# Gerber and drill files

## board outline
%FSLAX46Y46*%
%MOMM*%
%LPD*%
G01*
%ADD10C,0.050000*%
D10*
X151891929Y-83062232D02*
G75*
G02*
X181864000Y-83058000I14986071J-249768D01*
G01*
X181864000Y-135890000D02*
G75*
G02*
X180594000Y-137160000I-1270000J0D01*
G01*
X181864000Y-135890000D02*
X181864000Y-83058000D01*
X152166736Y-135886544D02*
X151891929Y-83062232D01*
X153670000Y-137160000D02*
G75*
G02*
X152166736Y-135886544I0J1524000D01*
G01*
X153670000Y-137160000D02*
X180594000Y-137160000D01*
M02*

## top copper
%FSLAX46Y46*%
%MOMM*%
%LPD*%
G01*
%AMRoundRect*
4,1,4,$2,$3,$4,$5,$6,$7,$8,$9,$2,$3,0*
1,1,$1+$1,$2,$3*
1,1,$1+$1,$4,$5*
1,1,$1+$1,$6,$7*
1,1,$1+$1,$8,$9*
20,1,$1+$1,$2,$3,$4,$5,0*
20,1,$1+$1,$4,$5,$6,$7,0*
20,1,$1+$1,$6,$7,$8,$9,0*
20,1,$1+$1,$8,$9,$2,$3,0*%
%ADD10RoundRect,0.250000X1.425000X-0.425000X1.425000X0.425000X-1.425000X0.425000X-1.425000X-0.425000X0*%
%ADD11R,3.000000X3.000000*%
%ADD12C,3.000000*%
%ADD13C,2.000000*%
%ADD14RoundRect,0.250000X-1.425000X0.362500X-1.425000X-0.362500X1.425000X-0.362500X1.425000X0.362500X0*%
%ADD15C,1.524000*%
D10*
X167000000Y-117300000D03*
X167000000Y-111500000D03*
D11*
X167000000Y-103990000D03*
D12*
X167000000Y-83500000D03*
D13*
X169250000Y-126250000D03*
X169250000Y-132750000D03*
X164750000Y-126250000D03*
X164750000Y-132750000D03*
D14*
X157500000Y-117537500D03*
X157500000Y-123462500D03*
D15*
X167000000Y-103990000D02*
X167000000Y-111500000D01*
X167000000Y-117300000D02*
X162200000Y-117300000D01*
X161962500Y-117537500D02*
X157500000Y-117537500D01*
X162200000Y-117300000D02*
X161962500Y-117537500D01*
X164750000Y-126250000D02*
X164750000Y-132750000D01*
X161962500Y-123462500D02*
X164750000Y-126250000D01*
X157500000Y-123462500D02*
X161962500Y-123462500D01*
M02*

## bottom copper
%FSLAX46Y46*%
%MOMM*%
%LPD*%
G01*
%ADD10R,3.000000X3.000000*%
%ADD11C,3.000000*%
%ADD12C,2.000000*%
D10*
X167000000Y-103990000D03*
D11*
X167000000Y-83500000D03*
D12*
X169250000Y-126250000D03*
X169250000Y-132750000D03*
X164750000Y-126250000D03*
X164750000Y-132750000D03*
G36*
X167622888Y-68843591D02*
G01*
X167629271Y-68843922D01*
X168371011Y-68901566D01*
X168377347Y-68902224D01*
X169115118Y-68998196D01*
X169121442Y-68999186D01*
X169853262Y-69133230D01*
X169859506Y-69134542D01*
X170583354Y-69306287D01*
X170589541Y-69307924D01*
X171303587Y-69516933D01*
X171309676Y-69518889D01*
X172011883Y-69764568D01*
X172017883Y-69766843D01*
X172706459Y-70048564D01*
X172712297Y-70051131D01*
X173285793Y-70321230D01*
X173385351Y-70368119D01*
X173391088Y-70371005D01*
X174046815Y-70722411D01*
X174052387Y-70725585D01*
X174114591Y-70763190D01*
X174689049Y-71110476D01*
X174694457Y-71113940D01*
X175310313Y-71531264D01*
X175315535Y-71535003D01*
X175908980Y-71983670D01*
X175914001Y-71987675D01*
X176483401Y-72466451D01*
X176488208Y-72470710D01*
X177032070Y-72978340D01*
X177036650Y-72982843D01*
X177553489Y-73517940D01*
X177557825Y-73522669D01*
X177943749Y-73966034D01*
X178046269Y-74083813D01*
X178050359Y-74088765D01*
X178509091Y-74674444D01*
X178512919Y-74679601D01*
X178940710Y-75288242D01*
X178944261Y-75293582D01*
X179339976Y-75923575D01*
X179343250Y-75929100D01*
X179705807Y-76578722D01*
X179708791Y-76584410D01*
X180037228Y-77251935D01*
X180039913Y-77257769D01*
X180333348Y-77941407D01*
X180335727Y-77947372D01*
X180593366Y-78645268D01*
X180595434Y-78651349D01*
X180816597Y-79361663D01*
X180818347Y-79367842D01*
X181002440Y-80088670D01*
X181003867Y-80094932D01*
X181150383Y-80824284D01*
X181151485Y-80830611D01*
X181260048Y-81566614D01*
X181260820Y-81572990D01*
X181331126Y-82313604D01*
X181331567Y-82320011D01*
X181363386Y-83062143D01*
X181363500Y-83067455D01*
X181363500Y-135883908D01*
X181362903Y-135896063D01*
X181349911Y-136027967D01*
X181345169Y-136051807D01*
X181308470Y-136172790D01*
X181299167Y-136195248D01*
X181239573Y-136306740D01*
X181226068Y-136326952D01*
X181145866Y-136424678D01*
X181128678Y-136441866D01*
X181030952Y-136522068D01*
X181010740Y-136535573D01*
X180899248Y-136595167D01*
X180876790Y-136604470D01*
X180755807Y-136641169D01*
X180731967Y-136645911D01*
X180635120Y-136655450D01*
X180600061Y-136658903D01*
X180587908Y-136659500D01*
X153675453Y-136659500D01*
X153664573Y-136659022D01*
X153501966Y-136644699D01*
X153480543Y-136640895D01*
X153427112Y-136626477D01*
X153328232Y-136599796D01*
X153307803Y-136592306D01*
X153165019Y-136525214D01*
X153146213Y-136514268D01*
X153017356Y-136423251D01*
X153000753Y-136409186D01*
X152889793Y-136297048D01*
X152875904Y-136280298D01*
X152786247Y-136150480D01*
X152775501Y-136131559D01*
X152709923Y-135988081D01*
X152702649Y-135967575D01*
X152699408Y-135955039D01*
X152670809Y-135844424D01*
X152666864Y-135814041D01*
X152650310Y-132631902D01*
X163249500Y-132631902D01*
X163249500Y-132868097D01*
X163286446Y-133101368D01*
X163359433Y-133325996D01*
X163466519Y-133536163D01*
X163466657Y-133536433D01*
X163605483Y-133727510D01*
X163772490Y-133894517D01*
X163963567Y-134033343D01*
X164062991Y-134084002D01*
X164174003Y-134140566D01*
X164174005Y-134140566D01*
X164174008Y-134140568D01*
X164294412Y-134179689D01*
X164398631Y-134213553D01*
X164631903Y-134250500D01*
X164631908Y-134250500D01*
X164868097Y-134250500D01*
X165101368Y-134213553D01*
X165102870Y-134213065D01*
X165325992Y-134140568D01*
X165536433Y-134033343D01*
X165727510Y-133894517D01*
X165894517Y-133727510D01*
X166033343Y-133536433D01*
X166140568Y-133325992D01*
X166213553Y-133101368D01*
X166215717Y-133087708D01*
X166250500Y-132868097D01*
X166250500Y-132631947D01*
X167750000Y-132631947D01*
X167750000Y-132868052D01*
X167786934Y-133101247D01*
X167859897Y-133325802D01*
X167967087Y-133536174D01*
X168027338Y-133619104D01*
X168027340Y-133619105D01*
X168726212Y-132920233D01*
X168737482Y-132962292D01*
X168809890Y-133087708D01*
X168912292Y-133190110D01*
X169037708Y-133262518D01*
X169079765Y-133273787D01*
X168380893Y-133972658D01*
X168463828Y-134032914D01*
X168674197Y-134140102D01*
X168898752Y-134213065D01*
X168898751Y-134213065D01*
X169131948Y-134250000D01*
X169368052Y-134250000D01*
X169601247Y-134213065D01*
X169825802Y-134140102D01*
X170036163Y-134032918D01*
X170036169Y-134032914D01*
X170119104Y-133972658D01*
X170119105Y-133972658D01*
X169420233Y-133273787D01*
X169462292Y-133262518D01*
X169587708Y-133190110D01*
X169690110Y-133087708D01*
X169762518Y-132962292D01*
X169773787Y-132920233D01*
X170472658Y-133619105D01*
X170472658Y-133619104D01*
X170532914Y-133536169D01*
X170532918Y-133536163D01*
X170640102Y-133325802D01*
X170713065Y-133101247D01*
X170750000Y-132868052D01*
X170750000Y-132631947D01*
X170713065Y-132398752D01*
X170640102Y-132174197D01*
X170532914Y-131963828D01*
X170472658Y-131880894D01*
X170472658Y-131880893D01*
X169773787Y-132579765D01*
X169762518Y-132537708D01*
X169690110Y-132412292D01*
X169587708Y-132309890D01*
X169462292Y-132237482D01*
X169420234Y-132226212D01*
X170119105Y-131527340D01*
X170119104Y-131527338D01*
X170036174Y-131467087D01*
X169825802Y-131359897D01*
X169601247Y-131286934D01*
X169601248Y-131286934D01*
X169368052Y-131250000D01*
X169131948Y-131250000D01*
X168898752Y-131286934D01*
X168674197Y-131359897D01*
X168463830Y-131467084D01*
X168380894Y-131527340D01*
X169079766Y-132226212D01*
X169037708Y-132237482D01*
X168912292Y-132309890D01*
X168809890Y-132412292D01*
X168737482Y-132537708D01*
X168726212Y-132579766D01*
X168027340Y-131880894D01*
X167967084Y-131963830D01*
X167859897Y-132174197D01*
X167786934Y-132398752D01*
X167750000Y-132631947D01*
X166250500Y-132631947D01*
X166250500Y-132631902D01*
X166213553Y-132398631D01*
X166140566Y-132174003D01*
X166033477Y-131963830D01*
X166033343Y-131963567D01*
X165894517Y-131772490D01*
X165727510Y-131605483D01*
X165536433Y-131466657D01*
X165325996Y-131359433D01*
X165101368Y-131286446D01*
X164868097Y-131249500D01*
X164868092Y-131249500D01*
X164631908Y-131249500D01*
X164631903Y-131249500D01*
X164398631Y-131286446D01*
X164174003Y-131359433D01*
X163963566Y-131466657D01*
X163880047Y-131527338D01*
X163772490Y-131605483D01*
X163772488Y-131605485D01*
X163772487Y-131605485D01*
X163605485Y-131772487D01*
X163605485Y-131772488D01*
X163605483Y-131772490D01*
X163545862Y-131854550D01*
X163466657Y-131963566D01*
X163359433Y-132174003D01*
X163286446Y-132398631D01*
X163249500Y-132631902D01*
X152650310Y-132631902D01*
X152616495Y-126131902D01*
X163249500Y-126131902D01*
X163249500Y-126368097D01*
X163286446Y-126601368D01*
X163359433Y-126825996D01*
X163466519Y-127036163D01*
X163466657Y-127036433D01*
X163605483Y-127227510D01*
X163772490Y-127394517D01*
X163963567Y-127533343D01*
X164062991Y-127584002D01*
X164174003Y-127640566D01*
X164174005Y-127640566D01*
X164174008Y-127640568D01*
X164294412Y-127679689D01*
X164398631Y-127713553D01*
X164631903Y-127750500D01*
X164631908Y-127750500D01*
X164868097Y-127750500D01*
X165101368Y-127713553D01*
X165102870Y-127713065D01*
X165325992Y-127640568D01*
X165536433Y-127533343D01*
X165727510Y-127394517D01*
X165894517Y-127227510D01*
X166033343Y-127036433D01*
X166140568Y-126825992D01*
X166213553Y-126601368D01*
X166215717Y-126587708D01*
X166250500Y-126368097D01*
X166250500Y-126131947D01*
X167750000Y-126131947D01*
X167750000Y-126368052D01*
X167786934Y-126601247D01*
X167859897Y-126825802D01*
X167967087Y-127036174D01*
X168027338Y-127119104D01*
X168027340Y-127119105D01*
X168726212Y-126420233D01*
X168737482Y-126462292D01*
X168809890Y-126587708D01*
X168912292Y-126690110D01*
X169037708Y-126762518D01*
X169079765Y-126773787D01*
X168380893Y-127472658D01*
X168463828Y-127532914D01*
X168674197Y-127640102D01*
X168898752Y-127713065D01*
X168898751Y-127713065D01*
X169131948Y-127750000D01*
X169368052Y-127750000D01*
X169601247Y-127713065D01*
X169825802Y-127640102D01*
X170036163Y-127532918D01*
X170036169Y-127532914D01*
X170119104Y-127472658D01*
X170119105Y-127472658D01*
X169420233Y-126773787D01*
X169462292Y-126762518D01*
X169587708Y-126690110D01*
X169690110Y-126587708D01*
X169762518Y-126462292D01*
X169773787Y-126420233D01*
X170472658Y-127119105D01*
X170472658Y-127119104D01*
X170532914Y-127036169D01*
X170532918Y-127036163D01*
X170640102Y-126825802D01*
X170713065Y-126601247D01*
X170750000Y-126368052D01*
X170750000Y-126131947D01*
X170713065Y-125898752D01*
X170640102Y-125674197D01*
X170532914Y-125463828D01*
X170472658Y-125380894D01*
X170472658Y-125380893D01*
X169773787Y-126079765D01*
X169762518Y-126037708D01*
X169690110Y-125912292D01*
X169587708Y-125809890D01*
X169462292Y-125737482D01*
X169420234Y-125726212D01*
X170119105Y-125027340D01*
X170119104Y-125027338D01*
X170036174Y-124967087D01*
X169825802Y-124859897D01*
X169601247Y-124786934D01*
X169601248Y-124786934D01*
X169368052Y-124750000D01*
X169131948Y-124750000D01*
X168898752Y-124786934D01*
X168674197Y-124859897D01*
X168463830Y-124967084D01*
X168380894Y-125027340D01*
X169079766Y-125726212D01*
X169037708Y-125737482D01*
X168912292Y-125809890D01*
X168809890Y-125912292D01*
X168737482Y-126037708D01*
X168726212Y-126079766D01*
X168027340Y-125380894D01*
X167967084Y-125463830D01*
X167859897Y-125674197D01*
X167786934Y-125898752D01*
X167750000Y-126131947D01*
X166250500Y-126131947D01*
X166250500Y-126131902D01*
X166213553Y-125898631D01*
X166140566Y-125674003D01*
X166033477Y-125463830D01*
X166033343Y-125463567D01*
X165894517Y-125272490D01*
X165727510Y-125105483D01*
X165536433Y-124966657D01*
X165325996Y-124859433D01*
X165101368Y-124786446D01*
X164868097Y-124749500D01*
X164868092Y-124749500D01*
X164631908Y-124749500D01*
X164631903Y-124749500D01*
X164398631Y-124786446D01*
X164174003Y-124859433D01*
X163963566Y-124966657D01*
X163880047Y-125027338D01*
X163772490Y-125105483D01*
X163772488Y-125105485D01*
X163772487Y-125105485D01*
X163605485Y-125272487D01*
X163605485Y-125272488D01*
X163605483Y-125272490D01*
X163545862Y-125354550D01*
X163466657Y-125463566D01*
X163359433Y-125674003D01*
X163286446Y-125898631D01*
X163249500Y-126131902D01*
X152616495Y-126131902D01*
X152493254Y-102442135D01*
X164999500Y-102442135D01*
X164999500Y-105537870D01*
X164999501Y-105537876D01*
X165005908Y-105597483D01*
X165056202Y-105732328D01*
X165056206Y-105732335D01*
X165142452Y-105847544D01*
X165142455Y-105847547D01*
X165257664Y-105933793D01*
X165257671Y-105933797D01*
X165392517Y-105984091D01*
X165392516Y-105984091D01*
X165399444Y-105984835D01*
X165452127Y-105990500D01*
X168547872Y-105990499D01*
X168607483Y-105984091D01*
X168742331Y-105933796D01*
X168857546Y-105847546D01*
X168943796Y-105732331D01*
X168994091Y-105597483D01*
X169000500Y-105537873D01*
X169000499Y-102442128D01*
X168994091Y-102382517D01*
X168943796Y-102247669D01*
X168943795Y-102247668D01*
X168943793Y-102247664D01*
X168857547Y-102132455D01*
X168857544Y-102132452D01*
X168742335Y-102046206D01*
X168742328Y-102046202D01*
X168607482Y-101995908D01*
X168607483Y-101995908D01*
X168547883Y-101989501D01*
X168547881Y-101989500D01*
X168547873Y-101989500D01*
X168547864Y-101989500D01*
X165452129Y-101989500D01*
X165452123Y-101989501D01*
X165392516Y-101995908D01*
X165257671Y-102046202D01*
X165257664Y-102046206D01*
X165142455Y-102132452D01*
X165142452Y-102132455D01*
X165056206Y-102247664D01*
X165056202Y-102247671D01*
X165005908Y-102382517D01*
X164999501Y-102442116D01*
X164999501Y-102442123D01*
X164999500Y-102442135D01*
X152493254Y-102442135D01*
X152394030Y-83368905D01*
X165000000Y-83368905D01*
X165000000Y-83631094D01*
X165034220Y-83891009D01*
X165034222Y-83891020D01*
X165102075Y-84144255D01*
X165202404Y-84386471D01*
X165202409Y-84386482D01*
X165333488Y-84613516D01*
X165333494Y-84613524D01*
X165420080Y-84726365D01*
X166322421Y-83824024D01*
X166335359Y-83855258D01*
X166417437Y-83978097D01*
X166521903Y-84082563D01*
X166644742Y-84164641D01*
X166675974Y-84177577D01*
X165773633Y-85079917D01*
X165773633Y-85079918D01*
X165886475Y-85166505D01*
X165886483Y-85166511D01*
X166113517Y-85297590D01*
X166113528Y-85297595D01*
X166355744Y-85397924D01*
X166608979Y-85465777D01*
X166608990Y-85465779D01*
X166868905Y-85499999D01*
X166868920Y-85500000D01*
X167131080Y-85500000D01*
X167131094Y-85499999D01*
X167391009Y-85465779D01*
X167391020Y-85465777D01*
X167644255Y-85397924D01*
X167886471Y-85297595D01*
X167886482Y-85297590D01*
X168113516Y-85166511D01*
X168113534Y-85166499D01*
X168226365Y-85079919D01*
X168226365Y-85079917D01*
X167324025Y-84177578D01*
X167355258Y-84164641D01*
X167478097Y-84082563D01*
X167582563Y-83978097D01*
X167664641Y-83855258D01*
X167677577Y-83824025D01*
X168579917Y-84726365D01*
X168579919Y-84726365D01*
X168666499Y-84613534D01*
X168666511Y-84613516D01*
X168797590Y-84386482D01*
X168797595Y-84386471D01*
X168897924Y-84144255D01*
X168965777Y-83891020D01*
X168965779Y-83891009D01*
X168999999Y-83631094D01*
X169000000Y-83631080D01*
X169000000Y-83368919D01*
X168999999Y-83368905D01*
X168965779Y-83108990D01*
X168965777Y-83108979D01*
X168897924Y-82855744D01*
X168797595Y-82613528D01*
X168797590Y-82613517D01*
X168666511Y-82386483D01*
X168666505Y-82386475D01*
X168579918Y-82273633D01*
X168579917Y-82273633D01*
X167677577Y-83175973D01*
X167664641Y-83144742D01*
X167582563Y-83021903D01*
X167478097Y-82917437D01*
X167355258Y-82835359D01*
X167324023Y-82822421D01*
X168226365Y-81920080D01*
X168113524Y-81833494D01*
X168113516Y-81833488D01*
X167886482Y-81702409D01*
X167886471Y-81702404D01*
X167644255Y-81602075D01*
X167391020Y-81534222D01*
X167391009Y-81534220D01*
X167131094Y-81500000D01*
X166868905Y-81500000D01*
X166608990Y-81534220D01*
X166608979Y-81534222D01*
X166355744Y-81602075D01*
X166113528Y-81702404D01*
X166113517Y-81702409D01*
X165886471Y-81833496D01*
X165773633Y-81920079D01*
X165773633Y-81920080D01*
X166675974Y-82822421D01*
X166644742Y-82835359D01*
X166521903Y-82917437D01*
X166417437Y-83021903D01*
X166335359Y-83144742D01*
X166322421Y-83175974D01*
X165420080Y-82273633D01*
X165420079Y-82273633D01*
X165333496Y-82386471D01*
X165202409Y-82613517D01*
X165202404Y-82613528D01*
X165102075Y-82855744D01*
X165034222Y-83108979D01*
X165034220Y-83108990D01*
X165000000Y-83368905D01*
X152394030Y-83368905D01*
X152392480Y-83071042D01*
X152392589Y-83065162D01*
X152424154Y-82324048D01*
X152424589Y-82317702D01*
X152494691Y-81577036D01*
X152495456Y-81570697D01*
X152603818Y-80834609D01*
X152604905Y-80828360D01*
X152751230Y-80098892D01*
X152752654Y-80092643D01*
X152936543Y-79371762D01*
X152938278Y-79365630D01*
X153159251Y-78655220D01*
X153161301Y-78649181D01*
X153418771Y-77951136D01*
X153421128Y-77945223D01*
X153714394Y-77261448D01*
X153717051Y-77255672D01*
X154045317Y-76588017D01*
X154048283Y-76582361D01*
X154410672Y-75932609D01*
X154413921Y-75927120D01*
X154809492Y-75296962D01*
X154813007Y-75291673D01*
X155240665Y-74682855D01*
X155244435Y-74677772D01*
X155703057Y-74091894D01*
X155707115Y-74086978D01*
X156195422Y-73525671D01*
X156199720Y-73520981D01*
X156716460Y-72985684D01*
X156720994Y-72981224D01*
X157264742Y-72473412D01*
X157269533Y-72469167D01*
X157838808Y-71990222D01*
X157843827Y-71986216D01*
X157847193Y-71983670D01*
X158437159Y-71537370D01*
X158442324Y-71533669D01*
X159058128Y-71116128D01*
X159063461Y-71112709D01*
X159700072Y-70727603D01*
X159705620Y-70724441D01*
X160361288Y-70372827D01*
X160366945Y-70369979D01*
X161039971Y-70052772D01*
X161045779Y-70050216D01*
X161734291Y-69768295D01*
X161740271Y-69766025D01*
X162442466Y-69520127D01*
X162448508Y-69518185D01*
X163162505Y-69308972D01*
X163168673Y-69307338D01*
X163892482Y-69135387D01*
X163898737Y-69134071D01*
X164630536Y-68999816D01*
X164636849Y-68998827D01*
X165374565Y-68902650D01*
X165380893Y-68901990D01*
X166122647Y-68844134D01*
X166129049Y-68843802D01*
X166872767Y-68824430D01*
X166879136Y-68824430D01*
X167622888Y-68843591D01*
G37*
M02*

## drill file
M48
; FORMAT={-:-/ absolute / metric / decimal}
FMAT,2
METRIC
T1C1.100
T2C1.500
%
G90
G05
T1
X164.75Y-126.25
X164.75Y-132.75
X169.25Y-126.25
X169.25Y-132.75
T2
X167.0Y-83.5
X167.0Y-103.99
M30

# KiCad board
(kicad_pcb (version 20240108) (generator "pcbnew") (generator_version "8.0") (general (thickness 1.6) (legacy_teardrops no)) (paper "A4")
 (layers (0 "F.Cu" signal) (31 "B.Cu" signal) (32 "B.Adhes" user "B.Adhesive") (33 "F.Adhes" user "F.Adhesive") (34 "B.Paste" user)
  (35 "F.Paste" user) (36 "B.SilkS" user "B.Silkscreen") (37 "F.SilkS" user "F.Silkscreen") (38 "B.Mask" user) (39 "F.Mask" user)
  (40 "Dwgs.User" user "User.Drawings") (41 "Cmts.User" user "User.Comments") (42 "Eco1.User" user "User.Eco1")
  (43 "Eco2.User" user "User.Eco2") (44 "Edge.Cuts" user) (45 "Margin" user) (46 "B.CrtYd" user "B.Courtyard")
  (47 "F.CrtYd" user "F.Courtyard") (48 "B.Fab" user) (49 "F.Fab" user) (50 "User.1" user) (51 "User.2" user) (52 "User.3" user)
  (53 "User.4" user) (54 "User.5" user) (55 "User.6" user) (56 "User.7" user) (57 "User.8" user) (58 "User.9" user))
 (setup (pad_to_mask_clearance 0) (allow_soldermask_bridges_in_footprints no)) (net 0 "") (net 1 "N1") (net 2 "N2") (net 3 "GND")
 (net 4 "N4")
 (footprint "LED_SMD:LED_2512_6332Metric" (layer "F.Cu") (at 167 114.4 90)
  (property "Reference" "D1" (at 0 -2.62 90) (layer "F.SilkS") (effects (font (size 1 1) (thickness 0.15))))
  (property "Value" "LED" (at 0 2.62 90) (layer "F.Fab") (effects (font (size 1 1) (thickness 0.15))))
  (pad "1" smd roundrect (at -2.9 0 90) (size 1.35 3.35) (layers "F.Cu" "F.Paste" "F.Mask") (roundrect_rratio 0.185185) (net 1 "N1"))
  (pad "2" smd roundrect (at 2.9 0 90) (size 1.35 3.35) (layers "F.Cu" "F.Paste" "F.Mask") (roundrect_rratio 0.185185) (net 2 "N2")))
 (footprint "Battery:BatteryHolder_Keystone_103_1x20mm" (layer "F.Cu") (at 167 103.99 90)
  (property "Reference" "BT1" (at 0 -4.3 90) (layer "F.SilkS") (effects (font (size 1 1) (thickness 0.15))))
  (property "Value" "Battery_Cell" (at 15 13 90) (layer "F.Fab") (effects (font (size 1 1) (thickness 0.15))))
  (pad "1" thru_hole rect (at 0 0 90) (size 3 3) (drill 1.5) (layers "*.Cu" "*.Mask") (remove_unused_layers no) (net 2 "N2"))
  (pad "2" thru_hole circle (at 20.49 0 90) (size 3 3) (drill 1.5) (layers "*.Cu" "*.Mask") (remove_unused_layers no) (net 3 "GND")))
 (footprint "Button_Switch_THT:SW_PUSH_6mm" (layer "F.Cu") (at 169.25 126.25 -90)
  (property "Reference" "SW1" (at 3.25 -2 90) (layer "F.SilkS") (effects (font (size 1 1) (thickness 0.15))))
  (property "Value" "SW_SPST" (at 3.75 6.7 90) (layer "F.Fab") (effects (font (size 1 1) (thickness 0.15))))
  (pad "1" thru_hole circle (at 0 0) (size 2 2) (drill 1.1) (layers "*.Cu" "*.Mask") (remove_unused_layers no) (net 3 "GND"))
  (pad "1" thru_hole circle (at 6.5 0) (size 2 2) (drill 1.1) (layers "*.Cu" "*.Mask") (remove_unused_layers no) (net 3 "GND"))
  (pad "2" thru_hole circle (at 0 4.5) (size 2 2) (drill 1.1) (layers "*.Cu" "*.Mask") (remove_unused_layers no) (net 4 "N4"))
  (pad "2" thru_hole circle (at 6.5 4.5) (size 2 2) (drill 1.1) (layers "*.Cu" "*.Mask") (remove_unused_layers no) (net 4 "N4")))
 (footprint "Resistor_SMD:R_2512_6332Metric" (layer "F.Cu") (at 157.5 120.5 -90)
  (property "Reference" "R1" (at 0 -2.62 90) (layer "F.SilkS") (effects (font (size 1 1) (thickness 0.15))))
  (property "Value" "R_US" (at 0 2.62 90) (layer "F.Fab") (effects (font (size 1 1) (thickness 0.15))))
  (pad "1" smd roundrect (at -2.9625 0 270) (size 1.225 3.35) (layers "F.Cu" "F.Paste" "F.Mask") (roundrect_rratio 0.204082) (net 1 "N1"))
  (pad "2" smd roundrect (at 2.9625 0 270) (size 1.225 3.35) (layers "F.Cu" "F.Paste" "F.Mask") (roundrect_rratio 0.204082) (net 4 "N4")))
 (gr_arc (start 151.891929 83.062232) (mid 166.875884 68.323848) (end 181.864 83.058) (stroke (width 0.05) (type default))
  (layer "Edge.Cuts"))
 (gr_arc (start 181.864 135.89) (mid 181.492026 136.788026) (end 180.594 137.16) (stroke (width 0.05) (type default)) (layer "Edge.Cuts"))
 (gr_line (start 181.864 135.89) (end 181.864 83.058) (stroke (width 0.05) (type default)) (layer "Edge.Cuts"))
 (gr_line (start 152.166736 135.886544) (end 151.891929 83.062232) (stroke (width 0.05) (type default)) (layer "Edge.Cuts"))
 (gr_arc (start 153.67 137.16) (mid 152.684925 136.798842) (end 152.166736 135.886544) (stroke (width 0.05) (type default))
  (layer "Edge.Cuts"))
 (gr_line (start 153.67 137.16) (end 180.594 137.16) (stroke (width 0.05) (type default)) (layer "Edge.Cuts"))
 (segment (start 167 103.99) (end 167 111.5) (width 1.524) (layer "F.Cu") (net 2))
 (segment (start 167 117.3) (end 162.2 117.3) (width 1.524) (layer "F.Cu") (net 1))
 (segment (start 161.9625 117.5375) (end 157.5 117.5375) (width 1.524) (layer "F.Cu") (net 1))
 (segment (start 162.2 117.3) (end 161.9625 117.5375) (width 1.524) (layer "F.Cu") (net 1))
 (segment (start 164.75 126.25) (end 164.75 132.75) (width 1.524) (layer "F.Cu") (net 4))
 (segment (start 161.9625 123.4625) (end 164.75 126.25) (width 1.524) (layer "F.Cu") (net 4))
 (segment (start 157.5 123.4625) (end 161.9625 123.4625) (width 1.524) (layer "F.Cu") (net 4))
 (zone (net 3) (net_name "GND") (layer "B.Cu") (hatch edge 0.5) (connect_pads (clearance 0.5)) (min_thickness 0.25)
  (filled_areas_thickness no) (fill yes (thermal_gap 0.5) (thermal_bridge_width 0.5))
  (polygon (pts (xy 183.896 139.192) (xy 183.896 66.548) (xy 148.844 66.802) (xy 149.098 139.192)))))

